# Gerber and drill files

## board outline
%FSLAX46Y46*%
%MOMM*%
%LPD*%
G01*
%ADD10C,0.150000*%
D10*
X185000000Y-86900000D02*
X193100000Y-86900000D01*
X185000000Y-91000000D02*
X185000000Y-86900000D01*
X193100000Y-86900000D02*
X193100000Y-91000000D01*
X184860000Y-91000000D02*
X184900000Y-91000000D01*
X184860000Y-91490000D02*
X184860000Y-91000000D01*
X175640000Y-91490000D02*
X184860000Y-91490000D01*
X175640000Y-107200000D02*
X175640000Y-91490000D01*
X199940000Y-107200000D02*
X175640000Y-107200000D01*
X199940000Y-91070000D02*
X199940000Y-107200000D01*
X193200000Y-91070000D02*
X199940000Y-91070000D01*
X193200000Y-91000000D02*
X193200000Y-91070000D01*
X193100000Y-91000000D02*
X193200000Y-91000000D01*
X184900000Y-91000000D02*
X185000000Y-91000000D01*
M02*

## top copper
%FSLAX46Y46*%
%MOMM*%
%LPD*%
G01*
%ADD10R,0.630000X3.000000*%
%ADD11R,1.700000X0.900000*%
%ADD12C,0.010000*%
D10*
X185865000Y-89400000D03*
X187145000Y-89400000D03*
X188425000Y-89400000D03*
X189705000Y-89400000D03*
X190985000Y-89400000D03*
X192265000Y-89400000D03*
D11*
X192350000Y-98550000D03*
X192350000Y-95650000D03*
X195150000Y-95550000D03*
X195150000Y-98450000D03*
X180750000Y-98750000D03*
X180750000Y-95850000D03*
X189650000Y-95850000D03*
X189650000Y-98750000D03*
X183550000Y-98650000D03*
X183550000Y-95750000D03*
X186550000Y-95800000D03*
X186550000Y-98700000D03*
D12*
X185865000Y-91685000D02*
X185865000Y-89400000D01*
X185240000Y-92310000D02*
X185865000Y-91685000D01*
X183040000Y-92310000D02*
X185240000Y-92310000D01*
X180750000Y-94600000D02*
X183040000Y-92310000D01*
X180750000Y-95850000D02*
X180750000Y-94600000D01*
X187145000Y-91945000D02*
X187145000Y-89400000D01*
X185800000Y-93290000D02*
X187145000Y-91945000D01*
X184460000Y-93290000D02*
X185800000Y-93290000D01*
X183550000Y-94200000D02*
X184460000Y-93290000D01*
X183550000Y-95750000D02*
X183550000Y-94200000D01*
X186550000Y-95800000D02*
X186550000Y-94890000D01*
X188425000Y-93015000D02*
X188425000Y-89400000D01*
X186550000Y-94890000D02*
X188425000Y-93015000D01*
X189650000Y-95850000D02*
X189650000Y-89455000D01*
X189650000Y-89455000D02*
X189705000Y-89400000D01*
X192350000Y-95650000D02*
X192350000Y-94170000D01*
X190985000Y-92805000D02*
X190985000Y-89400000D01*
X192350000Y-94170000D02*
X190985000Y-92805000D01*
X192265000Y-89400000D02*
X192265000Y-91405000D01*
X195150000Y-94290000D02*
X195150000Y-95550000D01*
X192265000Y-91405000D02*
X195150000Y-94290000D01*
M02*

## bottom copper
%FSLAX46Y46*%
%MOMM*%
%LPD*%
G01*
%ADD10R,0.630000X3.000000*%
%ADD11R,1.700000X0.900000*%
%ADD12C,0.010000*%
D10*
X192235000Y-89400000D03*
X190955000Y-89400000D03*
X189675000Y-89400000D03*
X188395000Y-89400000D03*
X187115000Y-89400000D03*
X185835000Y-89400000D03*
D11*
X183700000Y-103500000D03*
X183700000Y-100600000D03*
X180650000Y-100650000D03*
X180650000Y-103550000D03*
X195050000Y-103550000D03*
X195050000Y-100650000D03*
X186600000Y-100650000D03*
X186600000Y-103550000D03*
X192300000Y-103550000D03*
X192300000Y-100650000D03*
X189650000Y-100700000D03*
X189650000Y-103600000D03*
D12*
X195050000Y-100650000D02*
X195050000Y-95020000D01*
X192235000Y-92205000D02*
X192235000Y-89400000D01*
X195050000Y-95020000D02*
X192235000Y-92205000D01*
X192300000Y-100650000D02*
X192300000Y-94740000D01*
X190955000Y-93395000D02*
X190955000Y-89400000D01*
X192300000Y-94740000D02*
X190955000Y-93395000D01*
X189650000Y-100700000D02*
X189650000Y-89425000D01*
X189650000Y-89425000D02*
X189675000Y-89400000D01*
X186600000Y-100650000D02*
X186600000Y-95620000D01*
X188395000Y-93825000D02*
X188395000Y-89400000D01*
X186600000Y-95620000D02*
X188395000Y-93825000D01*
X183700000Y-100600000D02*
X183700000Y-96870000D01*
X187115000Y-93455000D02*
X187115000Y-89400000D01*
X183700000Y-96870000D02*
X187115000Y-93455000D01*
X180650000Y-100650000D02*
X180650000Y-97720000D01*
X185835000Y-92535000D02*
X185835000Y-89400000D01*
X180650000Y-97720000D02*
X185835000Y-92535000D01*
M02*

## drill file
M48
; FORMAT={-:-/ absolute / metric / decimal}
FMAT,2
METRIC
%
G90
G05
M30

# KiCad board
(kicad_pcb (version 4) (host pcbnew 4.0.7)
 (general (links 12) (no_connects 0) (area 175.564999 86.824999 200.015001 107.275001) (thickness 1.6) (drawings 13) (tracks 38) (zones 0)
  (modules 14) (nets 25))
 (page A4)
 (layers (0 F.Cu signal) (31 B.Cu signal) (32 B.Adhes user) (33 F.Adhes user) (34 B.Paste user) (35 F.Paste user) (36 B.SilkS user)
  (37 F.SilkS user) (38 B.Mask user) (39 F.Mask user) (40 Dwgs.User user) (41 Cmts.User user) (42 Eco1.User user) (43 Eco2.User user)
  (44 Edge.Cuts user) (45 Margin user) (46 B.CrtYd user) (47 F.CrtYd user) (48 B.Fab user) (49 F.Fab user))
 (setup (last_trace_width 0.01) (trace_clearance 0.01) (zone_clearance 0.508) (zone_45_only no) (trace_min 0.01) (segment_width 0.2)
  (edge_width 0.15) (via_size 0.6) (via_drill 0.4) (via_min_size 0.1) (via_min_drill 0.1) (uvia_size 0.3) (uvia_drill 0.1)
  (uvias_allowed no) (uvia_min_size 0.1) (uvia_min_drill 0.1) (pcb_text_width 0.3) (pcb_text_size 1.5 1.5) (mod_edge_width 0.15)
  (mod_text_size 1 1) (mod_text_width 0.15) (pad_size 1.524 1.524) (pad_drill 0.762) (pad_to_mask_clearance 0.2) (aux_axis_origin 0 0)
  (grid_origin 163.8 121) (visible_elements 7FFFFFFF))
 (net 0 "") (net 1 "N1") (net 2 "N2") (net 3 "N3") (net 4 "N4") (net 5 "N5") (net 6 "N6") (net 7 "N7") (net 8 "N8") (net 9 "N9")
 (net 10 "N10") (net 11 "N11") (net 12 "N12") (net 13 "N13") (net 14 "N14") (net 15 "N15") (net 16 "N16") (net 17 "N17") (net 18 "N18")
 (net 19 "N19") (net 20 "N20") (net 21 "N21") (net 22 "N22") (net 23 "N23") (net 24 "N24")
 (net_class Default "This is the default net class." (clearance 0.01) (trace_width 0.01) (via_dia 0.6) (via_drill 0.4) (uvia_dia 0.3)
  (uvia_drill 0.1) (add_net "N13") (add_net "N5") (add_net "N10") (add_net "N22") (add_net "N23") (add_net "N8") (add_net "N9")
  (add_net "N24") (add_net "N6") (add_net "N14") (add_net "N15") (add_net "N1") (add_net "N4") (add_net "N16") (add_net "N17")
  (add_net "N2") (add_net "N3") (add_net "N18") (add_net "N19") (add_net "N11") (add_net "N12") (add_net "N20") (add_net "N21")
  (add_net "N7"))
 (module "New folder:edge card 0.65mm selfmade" (layer F.Cu) (at 185 91)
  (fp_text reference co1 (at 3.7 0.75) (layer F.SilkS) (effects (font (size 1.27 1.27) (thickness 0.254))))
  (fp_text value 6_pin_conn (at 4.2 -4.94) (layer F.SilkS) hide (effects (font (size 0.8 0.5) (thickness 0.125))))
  (pad 1 connect rect (at 0.865 -1.6) (size 0.63 3) (layers F.Cu F.Mask) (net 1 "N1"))
  (pad 2 connect rect (at 2.145 -1.6) (size 0.63 3) (layers F.Cu F.Mask) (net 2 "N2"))
  (pad 3 connect rect (at 3.425 -1.6) (size 0.63 3) (layers F.Cu F.Mask) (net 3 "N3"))
  (pad 4 connect rect (at 4.705 -1.6) (size 0.63 3) (layers F.Cu F.Mask) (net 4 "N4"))
  (pad 5 connect rect (at 5.985 -1.6) (size 0.63 3) (layers F.Cu F.Mask) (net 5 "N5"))
  (pad 6 connect rect (at 7.265 -1.6) (size 0.63 3) (layers F.Cu F.Mask) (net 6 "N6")))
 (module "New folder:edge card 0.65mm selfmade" (layer B.Cu) (at 193.1 91 180)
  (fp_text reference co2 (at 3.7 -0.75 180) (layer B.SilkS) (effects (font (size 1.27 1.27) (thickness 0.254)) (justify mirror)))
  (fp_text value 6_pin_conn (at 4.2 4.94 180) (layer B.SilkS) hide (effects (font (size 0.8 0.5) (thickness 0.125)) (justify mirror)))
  (pad 1 connect rect (at 0.865 1.6 180) (size 0.63 3) (layers B.Cu B.Mask) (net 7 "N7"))
  (pad 2 connect rect (at 2.145 1.6 180) (size 0.63 3) (layers B.Cu B.Mask) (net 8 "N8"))
  (pad 3 connect rect (at 3.425 1.6 180) (size 0.63 3) (layers B.Cu B.Mask) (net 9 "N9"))
  (pad 4 connect rect (at 4.705 1.6 180) (size 0.63 3) (layers B.Cu B.Mask) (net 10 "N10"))
  (pad 5 connect rect (at 5.985 1.6 180) (size 0.63 3) (layers B.Cu B.Mask) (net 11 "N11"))
  (pad 6 connect rect (at 7.265 1.6 180) (size 0.63 3) (layers B.Cu B.Mask) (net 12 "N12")))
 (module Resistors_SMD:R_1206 (layer F.Cu) (at 192.35 97.1 90)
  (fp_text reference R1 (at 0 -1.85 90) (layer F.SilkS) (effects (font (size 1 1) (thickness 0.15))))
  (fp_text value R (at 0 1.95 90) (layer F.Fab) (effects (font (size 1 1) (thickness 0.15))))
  (pad 1 smd rect (at -1.45 0 90) (size 0.9 1.7) (layers F.Cu F.Paste F.Mask) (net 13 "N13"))
  (pad 2 smd rect (at 1.45 0 90) (size 0.9 1.7) (layers F.Cu F.Paste F.Mask) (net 5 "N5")))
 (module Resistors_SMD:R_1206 (layer F.Cu) (at 195.15 97 270)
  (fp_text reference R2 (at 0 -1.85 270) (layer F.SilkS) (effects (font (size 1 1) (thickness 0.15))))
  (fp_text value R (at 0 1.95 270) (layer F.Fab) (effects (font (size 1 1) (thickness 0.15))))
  (pad 1 smd rect (at -1.45 0 270) (size 0.9 1.7) (layers F.Cu F.Paste F.Mask) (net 6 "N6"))
  (pad 2 smd rect (at 1.45 0 270) (size 0.9 1.7) (layers F.Cu F.Paste F.Mask) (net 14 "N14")))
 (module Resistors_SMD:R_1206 (layer F.Cu) (at 180.75 97.3 90)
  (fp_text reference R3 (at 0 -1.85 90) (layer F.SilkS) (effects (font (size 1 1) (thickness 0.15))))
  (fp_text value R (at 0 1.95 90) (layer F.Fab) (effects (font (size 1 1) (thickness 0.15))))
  (pad 1 smd rect (at -1.45 0 90) (size 0.9 1.7) (layers F.Cu F.Paste F.Mask) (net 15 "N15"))
  (pad 2 smd rect (at 1.45 0 90) (size 0.9 1.7) (layers F.Cu F.Paste F.Mask) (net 1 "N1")))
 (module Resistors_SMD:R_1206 (layer F.Cu) (at 189.65 97.3 270)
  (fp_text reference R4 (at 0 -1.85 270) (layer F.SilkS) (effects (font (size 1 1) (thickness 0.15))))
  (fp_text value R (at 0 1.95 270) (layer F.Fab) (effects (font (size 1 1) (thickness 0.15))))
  (pad 1 smd rect (at -1.45 0 270) (size 0.9 1.7) (layers F.Cu F.Paste F.Mask) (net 4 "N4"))
  (pad 2 smd rect (at 1.45 0 270) (size 0.9 1.7) (layers F.Cu F.Paste F.Mask) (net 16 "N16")))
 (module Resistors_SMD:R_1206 (layer F.Cu) (at 183.55 97.2 90)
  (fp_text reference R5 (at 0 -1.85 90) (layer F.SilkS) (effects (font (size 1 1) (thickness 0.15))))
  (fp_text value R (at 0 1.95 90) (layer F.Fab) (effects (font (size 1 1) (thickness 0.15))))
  (pad 1 smd rect (at -1.45 0 90) (size 0.9 1.7) (layers F.Cu F.Paste F.Mask) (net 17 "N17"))
  (pad 2 smd rect (at 1.45 0 90) (size 0.9 1.7) (layers F.Cu F.Paste F.Mask) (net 2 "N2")))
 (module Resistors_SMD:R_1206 (layer F.Cu) (at 186.55 97.25 270)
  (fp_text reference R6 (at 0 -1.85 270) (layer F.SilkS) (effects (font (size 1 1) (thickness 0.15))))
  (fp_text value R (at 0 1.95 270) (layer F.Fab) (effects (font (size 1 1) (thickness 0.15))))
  (pad 1 smd rect (at -1.45 0 270) (size 0.9 1.7) (layers F.Cu F.Paste F.Mask) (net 3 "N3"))
  (pad 2 smd rect (at 1.45 0 270) (size 0.9 1.7) (layers F.Cu F.Paste F.Mask) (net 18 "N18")))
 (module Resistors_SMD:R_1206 (layer B.Cu) (at 183.7 102.05 90)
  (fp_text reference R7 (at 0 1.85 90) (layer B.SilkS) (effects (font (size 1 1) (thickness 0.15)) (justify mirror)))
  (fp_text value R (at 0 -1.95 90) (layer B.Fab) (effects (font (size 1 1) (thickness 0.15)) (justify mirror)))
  (pad 1 smd rect (at -1.45 0 90) (size 0.9 1.7) (layers B.Cu B.Paste B.Mask) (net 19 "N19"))
  (pad 2 smd rect (at 1.45 0 90) (size 0.9 1.7) (layers B.Cu B.Paste B.Mask) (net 11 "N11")))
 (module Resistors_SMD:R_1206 (layer B.Cu) (at 180.65 102.1 270)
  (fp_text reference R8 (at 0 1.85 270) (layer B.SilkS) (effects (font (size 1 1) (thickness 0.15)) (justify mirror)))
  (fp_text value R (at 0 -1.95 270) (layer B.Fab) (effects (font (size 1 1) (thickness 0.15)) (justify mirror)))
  (pad 1 smd rect (at -1.45 0 270) (size 0.9 1.7) (layers B.Cu B.Paste B.Mask) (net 12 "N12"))
  (pad 2 smd rect (at 1.45 0 270) (size 0.9 1.7) (layers B.Cu B.Paste B.Mask) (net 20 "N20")))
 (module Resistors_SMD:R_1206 (layer B.Cu) (at 195.05 102.1 90)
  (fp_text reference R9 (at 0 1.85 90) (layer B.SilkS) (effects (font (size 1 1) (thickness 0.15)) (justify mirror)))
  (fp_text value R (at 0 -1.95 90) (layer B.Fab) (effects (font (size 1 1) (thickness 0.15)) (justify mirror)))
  (pad 1 smd rect (at -1.45 0 90) (size 0.9 1.7) (layers B.Cu B.Paste B.Mask) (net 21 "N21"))
  (pad 2 smd rect (at 1.45 0 90) (size 0.9 1.7) (layers B.Cu B.Paste B.Mask) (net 7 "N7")))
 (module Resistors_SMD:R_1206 (layer B.Cu) (at 186.6 102.1 270)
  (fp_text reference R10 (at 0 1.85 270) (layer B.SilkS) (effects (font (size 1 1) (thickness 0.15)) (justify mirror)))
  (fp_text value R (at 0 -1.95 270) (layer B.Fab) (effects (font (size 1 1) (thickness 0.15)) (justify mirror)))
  (pad 1 smd rect (at -1.45 0 270) (size 0.9 1.7) (layers B.Cu B.Paste B.Mask) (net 10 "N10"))
  (pad 2 smd rect (at 1.45 0 270) (size 0.9 1.7) (layers B.Cu B.Paste B.Mask) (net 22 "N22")))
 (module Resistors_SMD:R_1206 (layer B.Cu) (at 192.3 102.1 90)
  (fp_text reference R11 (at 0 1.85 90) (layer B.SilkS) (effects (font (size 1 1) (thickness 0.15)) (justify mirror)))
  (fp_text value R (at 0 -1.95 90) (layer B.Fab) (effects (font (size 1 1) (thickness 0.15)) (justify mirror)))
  (pad 1 smd rect (at -1.45 0 90) (size 0.9 1.7) (layers B.Cu B.Paste B.Mask) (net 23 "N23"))
  (pad 2 smd rect (at 1.45 0 90) (size 0.9 1.7) (layers B.Cu B.Paste B.Mask) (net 8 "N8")))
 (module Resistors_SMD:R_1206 (layer B.Cu) (at 189.65 102.15 270)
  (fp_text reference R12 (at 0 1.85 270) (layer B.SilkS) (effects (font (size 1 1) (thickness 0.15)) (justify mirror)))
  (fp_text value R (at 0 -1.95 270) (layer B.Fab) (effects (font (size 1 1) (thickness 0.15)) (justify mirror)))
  (pad 1 smd rect (at -1.45 0 270) (size 0.9 1.7) (layers B.Cu B.Paste B.Mask) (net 9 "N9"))
  (pad 2 smd rect (at 1.45 0 270) (size 0.9 1.7) (layers B.Cu B.Paste B.Mask) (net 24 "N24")))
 (gr_line (start 185 86.9) (end 193.1 86.9) (angle 90) (layer Edge.Cuts) (width 0.15))
 (gr_line (start 185 91) (end 185 86.9) (angle 90) (layer Edge.Cuts) (width 0.15))
 (gr_line (start 193.1 86.9) (end 193.1 91) (angle 90) (layer Edge.Cuts) (width 0.15))
 (gr_line (start 184.86 91) (end 184.9 91) (angle 90) (layer Edge.Cuts) (width 0.15))
 (gr_line (start 184.86 91.49) (end 184.86 91) (angle 90) (layer Edge.Cuts) (width 0.15))
 (gr_line (start 175.64 91.49) (end 184.86 91.49) (angle 90) (layer Edge.Cuts) (width 0.15))
 (gr_line (start 175.64 107.2) (end 175.64 91.49) (angle 90) (layer Edge.Cuts) (width 0.15))
 (gr_line (start 199.94 107.2) (end 175.64 107.2) (angle 90) (layer Edge.Cuts) (width 0.15))
 (gr_line (start 199.94 91.07) (end 199.94 107.2) (angle 90) (layer Edge.Cuts) (width 0.15))
 (gr_line (start 193.2 91.07) (end 199.94 91.07) (angle 90) (layer Edge.Cuts) (width 0.15))
 (gr_line (start 193.2 91) (end 193.2 91.07) (angle 90) (layer Edge.Cuts) (width 0.15))
 (gr_line (start 193.1 91) (end 193.2 91) (angle 90) (layer Edge.Cuts) (width 0.15))
 (gr_line (start 184.9 91) (end 185 91) (angle 90) (layer Edge.Cuts) (width 0.15))
 (segment (start 185.865 91.685) (end 185.865 89.4) (width 0.01) (layer F.Cu) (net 1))
 (segment (start 185.24 92.31) (end 185.865 91.685) (width 0.01) (layer F.Cu) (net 1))
 (segment (start 183.04 92.31) (end 185.24 92.31) (width 0.01) (layer F.Cu) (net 1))
 (segment (start 180.75 94.6) (end 183.04 92.31) (width 0.01) (layer F.Cu) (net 1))
 (segment (start 180.75 95.85) (end 180.75 94.6) (width 0.01) (layer F.Cu) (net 1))
 (segment (start 187.145 91.945) (end 187.145 89.4) (width 0.01) (layer F.Cu) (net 2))
 (segment (start 185.8 93.29) (end 187.145 91.945) (width 0.01) (layer F.Cu) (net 2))
 (segment (start 184.46 93.29) (end 185.8 93.29) (width 0.01) (layer F.Cu) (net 2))
 (segment (start 183.55 94.2) (end 184.46 93.29) (width 0.01) (layer F.Cu) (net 2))
 (segment (start 183.55 95.75) (end 183.55 94.2) (width 0.01) (layer F.Cu) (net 2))
 (segment (start 186.55 95.8) (end 186.55 94.89) (width 0.01) (layer F.Cu) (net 3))
 (segment (start 188.425 93.015) (end 188.425 89.4) (width 0.01) (layer F.Cu) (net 3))
 (segment (start 186.55 94.89) (end 188.425 93.015) (width 0.01) (layer F.Cu) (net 3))
 (segment (start 189.65 95.85) (end 189.65 89.455) (width 0.01) (layer F.Cu) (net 4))
 (segment (start 189.65 89.455) (end 189.705 89.4) (width 0.01) (layer F.Cu) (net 4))
 (segment (start 192.35 95.65) (end 192.35 94.17) (width 0.01) (layer F.Cu) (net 5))
 (segment (start 190.985 92.805) (end 190.985 89.4) (width 0.01) (layer F.Cu) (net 5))
 (segment (start 192.35 94.17) (end 190.985 92.805) (width 0.01) (layer F.Cu) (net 5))
 (segment (start 192.265 89.4) (end 192.265 91.405) (width 0.01) (layer F.Cu) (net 6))
 (segment (start 195.15 94.29) (end 195.15 95.55) (width 0.01) (layer F.Cu) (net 6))
 (segment (start 192.265 91.405) (end 195.15 94.29) (width 0.01) (layer F.Cu) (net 6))
 (segment (start 195.05 100.65) (end 195.05 95.02) (width 0.01) (layer B.Cu) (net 7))
 (segment (start 192.235 92.205) (end 192.235 89.4) (width 0.01) (layer B.Cu) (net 7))
 (segment (start 195.05 95.02) (end 192.235 92.205) (width 0.01) (layer B.Cu) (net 7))
 (segment (start 192.3 100.65) (end 192.3 94.74) (width 0.01) (layer B.Cu) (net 8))
 (segment (start 190.955 93.395) (end 190.955 89.4) (width 0.01) (layer B.Cu) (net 8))
 (segment (start 192.3 94.74) (end 190.955 93.395) (width 0.01) (layer B.Cu) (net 8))
 (segment (start 189.65 100.7) (end 189.65 89.425) (width 0.01) (layer B.Cu) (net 9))
 (segment (start 189.65 89.425) (end 189.675 89.4) (width 0.01) (layer B.Cu) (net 9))
 (segment (start 186.6 100.65) (end 186.6 95.62) (width 0.01) (layer B.Cu) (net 10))
 (segment (start 188.395 93.825) (end 188.395 89.4) (width 0.01) (layer B.Cu) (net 10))
 (segment (start 186.6 95.62) (end 188.395 93.825) (width 0.01) (layer B.Cu) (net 10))
 (segment (start 183.7 100.6) (end 183.7 96.87) (width 0.01) (layer B.Cu) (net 11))
 (segment (start 187.115 93.455) (end 187.115 89.4) (width 0.01) (layer B.Cu) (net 11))
 (segment (start 183.7 96.87) (end 187.115 93.455) (width 0.01) (layer B.Cu) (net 11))
 (segment (start 180.65 100.65) (end 180.65 97.72) (width 0.01) (layer B.Cu) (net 12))
 (segment (start 185.835 92.535) (end 185.835 89.4) (width 0.01) (layer B.Cu) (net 12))
 (segment (start 180.65 97.72) (end 185.835 92.535) (width 0.01) (layer B.Cu) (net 12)))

